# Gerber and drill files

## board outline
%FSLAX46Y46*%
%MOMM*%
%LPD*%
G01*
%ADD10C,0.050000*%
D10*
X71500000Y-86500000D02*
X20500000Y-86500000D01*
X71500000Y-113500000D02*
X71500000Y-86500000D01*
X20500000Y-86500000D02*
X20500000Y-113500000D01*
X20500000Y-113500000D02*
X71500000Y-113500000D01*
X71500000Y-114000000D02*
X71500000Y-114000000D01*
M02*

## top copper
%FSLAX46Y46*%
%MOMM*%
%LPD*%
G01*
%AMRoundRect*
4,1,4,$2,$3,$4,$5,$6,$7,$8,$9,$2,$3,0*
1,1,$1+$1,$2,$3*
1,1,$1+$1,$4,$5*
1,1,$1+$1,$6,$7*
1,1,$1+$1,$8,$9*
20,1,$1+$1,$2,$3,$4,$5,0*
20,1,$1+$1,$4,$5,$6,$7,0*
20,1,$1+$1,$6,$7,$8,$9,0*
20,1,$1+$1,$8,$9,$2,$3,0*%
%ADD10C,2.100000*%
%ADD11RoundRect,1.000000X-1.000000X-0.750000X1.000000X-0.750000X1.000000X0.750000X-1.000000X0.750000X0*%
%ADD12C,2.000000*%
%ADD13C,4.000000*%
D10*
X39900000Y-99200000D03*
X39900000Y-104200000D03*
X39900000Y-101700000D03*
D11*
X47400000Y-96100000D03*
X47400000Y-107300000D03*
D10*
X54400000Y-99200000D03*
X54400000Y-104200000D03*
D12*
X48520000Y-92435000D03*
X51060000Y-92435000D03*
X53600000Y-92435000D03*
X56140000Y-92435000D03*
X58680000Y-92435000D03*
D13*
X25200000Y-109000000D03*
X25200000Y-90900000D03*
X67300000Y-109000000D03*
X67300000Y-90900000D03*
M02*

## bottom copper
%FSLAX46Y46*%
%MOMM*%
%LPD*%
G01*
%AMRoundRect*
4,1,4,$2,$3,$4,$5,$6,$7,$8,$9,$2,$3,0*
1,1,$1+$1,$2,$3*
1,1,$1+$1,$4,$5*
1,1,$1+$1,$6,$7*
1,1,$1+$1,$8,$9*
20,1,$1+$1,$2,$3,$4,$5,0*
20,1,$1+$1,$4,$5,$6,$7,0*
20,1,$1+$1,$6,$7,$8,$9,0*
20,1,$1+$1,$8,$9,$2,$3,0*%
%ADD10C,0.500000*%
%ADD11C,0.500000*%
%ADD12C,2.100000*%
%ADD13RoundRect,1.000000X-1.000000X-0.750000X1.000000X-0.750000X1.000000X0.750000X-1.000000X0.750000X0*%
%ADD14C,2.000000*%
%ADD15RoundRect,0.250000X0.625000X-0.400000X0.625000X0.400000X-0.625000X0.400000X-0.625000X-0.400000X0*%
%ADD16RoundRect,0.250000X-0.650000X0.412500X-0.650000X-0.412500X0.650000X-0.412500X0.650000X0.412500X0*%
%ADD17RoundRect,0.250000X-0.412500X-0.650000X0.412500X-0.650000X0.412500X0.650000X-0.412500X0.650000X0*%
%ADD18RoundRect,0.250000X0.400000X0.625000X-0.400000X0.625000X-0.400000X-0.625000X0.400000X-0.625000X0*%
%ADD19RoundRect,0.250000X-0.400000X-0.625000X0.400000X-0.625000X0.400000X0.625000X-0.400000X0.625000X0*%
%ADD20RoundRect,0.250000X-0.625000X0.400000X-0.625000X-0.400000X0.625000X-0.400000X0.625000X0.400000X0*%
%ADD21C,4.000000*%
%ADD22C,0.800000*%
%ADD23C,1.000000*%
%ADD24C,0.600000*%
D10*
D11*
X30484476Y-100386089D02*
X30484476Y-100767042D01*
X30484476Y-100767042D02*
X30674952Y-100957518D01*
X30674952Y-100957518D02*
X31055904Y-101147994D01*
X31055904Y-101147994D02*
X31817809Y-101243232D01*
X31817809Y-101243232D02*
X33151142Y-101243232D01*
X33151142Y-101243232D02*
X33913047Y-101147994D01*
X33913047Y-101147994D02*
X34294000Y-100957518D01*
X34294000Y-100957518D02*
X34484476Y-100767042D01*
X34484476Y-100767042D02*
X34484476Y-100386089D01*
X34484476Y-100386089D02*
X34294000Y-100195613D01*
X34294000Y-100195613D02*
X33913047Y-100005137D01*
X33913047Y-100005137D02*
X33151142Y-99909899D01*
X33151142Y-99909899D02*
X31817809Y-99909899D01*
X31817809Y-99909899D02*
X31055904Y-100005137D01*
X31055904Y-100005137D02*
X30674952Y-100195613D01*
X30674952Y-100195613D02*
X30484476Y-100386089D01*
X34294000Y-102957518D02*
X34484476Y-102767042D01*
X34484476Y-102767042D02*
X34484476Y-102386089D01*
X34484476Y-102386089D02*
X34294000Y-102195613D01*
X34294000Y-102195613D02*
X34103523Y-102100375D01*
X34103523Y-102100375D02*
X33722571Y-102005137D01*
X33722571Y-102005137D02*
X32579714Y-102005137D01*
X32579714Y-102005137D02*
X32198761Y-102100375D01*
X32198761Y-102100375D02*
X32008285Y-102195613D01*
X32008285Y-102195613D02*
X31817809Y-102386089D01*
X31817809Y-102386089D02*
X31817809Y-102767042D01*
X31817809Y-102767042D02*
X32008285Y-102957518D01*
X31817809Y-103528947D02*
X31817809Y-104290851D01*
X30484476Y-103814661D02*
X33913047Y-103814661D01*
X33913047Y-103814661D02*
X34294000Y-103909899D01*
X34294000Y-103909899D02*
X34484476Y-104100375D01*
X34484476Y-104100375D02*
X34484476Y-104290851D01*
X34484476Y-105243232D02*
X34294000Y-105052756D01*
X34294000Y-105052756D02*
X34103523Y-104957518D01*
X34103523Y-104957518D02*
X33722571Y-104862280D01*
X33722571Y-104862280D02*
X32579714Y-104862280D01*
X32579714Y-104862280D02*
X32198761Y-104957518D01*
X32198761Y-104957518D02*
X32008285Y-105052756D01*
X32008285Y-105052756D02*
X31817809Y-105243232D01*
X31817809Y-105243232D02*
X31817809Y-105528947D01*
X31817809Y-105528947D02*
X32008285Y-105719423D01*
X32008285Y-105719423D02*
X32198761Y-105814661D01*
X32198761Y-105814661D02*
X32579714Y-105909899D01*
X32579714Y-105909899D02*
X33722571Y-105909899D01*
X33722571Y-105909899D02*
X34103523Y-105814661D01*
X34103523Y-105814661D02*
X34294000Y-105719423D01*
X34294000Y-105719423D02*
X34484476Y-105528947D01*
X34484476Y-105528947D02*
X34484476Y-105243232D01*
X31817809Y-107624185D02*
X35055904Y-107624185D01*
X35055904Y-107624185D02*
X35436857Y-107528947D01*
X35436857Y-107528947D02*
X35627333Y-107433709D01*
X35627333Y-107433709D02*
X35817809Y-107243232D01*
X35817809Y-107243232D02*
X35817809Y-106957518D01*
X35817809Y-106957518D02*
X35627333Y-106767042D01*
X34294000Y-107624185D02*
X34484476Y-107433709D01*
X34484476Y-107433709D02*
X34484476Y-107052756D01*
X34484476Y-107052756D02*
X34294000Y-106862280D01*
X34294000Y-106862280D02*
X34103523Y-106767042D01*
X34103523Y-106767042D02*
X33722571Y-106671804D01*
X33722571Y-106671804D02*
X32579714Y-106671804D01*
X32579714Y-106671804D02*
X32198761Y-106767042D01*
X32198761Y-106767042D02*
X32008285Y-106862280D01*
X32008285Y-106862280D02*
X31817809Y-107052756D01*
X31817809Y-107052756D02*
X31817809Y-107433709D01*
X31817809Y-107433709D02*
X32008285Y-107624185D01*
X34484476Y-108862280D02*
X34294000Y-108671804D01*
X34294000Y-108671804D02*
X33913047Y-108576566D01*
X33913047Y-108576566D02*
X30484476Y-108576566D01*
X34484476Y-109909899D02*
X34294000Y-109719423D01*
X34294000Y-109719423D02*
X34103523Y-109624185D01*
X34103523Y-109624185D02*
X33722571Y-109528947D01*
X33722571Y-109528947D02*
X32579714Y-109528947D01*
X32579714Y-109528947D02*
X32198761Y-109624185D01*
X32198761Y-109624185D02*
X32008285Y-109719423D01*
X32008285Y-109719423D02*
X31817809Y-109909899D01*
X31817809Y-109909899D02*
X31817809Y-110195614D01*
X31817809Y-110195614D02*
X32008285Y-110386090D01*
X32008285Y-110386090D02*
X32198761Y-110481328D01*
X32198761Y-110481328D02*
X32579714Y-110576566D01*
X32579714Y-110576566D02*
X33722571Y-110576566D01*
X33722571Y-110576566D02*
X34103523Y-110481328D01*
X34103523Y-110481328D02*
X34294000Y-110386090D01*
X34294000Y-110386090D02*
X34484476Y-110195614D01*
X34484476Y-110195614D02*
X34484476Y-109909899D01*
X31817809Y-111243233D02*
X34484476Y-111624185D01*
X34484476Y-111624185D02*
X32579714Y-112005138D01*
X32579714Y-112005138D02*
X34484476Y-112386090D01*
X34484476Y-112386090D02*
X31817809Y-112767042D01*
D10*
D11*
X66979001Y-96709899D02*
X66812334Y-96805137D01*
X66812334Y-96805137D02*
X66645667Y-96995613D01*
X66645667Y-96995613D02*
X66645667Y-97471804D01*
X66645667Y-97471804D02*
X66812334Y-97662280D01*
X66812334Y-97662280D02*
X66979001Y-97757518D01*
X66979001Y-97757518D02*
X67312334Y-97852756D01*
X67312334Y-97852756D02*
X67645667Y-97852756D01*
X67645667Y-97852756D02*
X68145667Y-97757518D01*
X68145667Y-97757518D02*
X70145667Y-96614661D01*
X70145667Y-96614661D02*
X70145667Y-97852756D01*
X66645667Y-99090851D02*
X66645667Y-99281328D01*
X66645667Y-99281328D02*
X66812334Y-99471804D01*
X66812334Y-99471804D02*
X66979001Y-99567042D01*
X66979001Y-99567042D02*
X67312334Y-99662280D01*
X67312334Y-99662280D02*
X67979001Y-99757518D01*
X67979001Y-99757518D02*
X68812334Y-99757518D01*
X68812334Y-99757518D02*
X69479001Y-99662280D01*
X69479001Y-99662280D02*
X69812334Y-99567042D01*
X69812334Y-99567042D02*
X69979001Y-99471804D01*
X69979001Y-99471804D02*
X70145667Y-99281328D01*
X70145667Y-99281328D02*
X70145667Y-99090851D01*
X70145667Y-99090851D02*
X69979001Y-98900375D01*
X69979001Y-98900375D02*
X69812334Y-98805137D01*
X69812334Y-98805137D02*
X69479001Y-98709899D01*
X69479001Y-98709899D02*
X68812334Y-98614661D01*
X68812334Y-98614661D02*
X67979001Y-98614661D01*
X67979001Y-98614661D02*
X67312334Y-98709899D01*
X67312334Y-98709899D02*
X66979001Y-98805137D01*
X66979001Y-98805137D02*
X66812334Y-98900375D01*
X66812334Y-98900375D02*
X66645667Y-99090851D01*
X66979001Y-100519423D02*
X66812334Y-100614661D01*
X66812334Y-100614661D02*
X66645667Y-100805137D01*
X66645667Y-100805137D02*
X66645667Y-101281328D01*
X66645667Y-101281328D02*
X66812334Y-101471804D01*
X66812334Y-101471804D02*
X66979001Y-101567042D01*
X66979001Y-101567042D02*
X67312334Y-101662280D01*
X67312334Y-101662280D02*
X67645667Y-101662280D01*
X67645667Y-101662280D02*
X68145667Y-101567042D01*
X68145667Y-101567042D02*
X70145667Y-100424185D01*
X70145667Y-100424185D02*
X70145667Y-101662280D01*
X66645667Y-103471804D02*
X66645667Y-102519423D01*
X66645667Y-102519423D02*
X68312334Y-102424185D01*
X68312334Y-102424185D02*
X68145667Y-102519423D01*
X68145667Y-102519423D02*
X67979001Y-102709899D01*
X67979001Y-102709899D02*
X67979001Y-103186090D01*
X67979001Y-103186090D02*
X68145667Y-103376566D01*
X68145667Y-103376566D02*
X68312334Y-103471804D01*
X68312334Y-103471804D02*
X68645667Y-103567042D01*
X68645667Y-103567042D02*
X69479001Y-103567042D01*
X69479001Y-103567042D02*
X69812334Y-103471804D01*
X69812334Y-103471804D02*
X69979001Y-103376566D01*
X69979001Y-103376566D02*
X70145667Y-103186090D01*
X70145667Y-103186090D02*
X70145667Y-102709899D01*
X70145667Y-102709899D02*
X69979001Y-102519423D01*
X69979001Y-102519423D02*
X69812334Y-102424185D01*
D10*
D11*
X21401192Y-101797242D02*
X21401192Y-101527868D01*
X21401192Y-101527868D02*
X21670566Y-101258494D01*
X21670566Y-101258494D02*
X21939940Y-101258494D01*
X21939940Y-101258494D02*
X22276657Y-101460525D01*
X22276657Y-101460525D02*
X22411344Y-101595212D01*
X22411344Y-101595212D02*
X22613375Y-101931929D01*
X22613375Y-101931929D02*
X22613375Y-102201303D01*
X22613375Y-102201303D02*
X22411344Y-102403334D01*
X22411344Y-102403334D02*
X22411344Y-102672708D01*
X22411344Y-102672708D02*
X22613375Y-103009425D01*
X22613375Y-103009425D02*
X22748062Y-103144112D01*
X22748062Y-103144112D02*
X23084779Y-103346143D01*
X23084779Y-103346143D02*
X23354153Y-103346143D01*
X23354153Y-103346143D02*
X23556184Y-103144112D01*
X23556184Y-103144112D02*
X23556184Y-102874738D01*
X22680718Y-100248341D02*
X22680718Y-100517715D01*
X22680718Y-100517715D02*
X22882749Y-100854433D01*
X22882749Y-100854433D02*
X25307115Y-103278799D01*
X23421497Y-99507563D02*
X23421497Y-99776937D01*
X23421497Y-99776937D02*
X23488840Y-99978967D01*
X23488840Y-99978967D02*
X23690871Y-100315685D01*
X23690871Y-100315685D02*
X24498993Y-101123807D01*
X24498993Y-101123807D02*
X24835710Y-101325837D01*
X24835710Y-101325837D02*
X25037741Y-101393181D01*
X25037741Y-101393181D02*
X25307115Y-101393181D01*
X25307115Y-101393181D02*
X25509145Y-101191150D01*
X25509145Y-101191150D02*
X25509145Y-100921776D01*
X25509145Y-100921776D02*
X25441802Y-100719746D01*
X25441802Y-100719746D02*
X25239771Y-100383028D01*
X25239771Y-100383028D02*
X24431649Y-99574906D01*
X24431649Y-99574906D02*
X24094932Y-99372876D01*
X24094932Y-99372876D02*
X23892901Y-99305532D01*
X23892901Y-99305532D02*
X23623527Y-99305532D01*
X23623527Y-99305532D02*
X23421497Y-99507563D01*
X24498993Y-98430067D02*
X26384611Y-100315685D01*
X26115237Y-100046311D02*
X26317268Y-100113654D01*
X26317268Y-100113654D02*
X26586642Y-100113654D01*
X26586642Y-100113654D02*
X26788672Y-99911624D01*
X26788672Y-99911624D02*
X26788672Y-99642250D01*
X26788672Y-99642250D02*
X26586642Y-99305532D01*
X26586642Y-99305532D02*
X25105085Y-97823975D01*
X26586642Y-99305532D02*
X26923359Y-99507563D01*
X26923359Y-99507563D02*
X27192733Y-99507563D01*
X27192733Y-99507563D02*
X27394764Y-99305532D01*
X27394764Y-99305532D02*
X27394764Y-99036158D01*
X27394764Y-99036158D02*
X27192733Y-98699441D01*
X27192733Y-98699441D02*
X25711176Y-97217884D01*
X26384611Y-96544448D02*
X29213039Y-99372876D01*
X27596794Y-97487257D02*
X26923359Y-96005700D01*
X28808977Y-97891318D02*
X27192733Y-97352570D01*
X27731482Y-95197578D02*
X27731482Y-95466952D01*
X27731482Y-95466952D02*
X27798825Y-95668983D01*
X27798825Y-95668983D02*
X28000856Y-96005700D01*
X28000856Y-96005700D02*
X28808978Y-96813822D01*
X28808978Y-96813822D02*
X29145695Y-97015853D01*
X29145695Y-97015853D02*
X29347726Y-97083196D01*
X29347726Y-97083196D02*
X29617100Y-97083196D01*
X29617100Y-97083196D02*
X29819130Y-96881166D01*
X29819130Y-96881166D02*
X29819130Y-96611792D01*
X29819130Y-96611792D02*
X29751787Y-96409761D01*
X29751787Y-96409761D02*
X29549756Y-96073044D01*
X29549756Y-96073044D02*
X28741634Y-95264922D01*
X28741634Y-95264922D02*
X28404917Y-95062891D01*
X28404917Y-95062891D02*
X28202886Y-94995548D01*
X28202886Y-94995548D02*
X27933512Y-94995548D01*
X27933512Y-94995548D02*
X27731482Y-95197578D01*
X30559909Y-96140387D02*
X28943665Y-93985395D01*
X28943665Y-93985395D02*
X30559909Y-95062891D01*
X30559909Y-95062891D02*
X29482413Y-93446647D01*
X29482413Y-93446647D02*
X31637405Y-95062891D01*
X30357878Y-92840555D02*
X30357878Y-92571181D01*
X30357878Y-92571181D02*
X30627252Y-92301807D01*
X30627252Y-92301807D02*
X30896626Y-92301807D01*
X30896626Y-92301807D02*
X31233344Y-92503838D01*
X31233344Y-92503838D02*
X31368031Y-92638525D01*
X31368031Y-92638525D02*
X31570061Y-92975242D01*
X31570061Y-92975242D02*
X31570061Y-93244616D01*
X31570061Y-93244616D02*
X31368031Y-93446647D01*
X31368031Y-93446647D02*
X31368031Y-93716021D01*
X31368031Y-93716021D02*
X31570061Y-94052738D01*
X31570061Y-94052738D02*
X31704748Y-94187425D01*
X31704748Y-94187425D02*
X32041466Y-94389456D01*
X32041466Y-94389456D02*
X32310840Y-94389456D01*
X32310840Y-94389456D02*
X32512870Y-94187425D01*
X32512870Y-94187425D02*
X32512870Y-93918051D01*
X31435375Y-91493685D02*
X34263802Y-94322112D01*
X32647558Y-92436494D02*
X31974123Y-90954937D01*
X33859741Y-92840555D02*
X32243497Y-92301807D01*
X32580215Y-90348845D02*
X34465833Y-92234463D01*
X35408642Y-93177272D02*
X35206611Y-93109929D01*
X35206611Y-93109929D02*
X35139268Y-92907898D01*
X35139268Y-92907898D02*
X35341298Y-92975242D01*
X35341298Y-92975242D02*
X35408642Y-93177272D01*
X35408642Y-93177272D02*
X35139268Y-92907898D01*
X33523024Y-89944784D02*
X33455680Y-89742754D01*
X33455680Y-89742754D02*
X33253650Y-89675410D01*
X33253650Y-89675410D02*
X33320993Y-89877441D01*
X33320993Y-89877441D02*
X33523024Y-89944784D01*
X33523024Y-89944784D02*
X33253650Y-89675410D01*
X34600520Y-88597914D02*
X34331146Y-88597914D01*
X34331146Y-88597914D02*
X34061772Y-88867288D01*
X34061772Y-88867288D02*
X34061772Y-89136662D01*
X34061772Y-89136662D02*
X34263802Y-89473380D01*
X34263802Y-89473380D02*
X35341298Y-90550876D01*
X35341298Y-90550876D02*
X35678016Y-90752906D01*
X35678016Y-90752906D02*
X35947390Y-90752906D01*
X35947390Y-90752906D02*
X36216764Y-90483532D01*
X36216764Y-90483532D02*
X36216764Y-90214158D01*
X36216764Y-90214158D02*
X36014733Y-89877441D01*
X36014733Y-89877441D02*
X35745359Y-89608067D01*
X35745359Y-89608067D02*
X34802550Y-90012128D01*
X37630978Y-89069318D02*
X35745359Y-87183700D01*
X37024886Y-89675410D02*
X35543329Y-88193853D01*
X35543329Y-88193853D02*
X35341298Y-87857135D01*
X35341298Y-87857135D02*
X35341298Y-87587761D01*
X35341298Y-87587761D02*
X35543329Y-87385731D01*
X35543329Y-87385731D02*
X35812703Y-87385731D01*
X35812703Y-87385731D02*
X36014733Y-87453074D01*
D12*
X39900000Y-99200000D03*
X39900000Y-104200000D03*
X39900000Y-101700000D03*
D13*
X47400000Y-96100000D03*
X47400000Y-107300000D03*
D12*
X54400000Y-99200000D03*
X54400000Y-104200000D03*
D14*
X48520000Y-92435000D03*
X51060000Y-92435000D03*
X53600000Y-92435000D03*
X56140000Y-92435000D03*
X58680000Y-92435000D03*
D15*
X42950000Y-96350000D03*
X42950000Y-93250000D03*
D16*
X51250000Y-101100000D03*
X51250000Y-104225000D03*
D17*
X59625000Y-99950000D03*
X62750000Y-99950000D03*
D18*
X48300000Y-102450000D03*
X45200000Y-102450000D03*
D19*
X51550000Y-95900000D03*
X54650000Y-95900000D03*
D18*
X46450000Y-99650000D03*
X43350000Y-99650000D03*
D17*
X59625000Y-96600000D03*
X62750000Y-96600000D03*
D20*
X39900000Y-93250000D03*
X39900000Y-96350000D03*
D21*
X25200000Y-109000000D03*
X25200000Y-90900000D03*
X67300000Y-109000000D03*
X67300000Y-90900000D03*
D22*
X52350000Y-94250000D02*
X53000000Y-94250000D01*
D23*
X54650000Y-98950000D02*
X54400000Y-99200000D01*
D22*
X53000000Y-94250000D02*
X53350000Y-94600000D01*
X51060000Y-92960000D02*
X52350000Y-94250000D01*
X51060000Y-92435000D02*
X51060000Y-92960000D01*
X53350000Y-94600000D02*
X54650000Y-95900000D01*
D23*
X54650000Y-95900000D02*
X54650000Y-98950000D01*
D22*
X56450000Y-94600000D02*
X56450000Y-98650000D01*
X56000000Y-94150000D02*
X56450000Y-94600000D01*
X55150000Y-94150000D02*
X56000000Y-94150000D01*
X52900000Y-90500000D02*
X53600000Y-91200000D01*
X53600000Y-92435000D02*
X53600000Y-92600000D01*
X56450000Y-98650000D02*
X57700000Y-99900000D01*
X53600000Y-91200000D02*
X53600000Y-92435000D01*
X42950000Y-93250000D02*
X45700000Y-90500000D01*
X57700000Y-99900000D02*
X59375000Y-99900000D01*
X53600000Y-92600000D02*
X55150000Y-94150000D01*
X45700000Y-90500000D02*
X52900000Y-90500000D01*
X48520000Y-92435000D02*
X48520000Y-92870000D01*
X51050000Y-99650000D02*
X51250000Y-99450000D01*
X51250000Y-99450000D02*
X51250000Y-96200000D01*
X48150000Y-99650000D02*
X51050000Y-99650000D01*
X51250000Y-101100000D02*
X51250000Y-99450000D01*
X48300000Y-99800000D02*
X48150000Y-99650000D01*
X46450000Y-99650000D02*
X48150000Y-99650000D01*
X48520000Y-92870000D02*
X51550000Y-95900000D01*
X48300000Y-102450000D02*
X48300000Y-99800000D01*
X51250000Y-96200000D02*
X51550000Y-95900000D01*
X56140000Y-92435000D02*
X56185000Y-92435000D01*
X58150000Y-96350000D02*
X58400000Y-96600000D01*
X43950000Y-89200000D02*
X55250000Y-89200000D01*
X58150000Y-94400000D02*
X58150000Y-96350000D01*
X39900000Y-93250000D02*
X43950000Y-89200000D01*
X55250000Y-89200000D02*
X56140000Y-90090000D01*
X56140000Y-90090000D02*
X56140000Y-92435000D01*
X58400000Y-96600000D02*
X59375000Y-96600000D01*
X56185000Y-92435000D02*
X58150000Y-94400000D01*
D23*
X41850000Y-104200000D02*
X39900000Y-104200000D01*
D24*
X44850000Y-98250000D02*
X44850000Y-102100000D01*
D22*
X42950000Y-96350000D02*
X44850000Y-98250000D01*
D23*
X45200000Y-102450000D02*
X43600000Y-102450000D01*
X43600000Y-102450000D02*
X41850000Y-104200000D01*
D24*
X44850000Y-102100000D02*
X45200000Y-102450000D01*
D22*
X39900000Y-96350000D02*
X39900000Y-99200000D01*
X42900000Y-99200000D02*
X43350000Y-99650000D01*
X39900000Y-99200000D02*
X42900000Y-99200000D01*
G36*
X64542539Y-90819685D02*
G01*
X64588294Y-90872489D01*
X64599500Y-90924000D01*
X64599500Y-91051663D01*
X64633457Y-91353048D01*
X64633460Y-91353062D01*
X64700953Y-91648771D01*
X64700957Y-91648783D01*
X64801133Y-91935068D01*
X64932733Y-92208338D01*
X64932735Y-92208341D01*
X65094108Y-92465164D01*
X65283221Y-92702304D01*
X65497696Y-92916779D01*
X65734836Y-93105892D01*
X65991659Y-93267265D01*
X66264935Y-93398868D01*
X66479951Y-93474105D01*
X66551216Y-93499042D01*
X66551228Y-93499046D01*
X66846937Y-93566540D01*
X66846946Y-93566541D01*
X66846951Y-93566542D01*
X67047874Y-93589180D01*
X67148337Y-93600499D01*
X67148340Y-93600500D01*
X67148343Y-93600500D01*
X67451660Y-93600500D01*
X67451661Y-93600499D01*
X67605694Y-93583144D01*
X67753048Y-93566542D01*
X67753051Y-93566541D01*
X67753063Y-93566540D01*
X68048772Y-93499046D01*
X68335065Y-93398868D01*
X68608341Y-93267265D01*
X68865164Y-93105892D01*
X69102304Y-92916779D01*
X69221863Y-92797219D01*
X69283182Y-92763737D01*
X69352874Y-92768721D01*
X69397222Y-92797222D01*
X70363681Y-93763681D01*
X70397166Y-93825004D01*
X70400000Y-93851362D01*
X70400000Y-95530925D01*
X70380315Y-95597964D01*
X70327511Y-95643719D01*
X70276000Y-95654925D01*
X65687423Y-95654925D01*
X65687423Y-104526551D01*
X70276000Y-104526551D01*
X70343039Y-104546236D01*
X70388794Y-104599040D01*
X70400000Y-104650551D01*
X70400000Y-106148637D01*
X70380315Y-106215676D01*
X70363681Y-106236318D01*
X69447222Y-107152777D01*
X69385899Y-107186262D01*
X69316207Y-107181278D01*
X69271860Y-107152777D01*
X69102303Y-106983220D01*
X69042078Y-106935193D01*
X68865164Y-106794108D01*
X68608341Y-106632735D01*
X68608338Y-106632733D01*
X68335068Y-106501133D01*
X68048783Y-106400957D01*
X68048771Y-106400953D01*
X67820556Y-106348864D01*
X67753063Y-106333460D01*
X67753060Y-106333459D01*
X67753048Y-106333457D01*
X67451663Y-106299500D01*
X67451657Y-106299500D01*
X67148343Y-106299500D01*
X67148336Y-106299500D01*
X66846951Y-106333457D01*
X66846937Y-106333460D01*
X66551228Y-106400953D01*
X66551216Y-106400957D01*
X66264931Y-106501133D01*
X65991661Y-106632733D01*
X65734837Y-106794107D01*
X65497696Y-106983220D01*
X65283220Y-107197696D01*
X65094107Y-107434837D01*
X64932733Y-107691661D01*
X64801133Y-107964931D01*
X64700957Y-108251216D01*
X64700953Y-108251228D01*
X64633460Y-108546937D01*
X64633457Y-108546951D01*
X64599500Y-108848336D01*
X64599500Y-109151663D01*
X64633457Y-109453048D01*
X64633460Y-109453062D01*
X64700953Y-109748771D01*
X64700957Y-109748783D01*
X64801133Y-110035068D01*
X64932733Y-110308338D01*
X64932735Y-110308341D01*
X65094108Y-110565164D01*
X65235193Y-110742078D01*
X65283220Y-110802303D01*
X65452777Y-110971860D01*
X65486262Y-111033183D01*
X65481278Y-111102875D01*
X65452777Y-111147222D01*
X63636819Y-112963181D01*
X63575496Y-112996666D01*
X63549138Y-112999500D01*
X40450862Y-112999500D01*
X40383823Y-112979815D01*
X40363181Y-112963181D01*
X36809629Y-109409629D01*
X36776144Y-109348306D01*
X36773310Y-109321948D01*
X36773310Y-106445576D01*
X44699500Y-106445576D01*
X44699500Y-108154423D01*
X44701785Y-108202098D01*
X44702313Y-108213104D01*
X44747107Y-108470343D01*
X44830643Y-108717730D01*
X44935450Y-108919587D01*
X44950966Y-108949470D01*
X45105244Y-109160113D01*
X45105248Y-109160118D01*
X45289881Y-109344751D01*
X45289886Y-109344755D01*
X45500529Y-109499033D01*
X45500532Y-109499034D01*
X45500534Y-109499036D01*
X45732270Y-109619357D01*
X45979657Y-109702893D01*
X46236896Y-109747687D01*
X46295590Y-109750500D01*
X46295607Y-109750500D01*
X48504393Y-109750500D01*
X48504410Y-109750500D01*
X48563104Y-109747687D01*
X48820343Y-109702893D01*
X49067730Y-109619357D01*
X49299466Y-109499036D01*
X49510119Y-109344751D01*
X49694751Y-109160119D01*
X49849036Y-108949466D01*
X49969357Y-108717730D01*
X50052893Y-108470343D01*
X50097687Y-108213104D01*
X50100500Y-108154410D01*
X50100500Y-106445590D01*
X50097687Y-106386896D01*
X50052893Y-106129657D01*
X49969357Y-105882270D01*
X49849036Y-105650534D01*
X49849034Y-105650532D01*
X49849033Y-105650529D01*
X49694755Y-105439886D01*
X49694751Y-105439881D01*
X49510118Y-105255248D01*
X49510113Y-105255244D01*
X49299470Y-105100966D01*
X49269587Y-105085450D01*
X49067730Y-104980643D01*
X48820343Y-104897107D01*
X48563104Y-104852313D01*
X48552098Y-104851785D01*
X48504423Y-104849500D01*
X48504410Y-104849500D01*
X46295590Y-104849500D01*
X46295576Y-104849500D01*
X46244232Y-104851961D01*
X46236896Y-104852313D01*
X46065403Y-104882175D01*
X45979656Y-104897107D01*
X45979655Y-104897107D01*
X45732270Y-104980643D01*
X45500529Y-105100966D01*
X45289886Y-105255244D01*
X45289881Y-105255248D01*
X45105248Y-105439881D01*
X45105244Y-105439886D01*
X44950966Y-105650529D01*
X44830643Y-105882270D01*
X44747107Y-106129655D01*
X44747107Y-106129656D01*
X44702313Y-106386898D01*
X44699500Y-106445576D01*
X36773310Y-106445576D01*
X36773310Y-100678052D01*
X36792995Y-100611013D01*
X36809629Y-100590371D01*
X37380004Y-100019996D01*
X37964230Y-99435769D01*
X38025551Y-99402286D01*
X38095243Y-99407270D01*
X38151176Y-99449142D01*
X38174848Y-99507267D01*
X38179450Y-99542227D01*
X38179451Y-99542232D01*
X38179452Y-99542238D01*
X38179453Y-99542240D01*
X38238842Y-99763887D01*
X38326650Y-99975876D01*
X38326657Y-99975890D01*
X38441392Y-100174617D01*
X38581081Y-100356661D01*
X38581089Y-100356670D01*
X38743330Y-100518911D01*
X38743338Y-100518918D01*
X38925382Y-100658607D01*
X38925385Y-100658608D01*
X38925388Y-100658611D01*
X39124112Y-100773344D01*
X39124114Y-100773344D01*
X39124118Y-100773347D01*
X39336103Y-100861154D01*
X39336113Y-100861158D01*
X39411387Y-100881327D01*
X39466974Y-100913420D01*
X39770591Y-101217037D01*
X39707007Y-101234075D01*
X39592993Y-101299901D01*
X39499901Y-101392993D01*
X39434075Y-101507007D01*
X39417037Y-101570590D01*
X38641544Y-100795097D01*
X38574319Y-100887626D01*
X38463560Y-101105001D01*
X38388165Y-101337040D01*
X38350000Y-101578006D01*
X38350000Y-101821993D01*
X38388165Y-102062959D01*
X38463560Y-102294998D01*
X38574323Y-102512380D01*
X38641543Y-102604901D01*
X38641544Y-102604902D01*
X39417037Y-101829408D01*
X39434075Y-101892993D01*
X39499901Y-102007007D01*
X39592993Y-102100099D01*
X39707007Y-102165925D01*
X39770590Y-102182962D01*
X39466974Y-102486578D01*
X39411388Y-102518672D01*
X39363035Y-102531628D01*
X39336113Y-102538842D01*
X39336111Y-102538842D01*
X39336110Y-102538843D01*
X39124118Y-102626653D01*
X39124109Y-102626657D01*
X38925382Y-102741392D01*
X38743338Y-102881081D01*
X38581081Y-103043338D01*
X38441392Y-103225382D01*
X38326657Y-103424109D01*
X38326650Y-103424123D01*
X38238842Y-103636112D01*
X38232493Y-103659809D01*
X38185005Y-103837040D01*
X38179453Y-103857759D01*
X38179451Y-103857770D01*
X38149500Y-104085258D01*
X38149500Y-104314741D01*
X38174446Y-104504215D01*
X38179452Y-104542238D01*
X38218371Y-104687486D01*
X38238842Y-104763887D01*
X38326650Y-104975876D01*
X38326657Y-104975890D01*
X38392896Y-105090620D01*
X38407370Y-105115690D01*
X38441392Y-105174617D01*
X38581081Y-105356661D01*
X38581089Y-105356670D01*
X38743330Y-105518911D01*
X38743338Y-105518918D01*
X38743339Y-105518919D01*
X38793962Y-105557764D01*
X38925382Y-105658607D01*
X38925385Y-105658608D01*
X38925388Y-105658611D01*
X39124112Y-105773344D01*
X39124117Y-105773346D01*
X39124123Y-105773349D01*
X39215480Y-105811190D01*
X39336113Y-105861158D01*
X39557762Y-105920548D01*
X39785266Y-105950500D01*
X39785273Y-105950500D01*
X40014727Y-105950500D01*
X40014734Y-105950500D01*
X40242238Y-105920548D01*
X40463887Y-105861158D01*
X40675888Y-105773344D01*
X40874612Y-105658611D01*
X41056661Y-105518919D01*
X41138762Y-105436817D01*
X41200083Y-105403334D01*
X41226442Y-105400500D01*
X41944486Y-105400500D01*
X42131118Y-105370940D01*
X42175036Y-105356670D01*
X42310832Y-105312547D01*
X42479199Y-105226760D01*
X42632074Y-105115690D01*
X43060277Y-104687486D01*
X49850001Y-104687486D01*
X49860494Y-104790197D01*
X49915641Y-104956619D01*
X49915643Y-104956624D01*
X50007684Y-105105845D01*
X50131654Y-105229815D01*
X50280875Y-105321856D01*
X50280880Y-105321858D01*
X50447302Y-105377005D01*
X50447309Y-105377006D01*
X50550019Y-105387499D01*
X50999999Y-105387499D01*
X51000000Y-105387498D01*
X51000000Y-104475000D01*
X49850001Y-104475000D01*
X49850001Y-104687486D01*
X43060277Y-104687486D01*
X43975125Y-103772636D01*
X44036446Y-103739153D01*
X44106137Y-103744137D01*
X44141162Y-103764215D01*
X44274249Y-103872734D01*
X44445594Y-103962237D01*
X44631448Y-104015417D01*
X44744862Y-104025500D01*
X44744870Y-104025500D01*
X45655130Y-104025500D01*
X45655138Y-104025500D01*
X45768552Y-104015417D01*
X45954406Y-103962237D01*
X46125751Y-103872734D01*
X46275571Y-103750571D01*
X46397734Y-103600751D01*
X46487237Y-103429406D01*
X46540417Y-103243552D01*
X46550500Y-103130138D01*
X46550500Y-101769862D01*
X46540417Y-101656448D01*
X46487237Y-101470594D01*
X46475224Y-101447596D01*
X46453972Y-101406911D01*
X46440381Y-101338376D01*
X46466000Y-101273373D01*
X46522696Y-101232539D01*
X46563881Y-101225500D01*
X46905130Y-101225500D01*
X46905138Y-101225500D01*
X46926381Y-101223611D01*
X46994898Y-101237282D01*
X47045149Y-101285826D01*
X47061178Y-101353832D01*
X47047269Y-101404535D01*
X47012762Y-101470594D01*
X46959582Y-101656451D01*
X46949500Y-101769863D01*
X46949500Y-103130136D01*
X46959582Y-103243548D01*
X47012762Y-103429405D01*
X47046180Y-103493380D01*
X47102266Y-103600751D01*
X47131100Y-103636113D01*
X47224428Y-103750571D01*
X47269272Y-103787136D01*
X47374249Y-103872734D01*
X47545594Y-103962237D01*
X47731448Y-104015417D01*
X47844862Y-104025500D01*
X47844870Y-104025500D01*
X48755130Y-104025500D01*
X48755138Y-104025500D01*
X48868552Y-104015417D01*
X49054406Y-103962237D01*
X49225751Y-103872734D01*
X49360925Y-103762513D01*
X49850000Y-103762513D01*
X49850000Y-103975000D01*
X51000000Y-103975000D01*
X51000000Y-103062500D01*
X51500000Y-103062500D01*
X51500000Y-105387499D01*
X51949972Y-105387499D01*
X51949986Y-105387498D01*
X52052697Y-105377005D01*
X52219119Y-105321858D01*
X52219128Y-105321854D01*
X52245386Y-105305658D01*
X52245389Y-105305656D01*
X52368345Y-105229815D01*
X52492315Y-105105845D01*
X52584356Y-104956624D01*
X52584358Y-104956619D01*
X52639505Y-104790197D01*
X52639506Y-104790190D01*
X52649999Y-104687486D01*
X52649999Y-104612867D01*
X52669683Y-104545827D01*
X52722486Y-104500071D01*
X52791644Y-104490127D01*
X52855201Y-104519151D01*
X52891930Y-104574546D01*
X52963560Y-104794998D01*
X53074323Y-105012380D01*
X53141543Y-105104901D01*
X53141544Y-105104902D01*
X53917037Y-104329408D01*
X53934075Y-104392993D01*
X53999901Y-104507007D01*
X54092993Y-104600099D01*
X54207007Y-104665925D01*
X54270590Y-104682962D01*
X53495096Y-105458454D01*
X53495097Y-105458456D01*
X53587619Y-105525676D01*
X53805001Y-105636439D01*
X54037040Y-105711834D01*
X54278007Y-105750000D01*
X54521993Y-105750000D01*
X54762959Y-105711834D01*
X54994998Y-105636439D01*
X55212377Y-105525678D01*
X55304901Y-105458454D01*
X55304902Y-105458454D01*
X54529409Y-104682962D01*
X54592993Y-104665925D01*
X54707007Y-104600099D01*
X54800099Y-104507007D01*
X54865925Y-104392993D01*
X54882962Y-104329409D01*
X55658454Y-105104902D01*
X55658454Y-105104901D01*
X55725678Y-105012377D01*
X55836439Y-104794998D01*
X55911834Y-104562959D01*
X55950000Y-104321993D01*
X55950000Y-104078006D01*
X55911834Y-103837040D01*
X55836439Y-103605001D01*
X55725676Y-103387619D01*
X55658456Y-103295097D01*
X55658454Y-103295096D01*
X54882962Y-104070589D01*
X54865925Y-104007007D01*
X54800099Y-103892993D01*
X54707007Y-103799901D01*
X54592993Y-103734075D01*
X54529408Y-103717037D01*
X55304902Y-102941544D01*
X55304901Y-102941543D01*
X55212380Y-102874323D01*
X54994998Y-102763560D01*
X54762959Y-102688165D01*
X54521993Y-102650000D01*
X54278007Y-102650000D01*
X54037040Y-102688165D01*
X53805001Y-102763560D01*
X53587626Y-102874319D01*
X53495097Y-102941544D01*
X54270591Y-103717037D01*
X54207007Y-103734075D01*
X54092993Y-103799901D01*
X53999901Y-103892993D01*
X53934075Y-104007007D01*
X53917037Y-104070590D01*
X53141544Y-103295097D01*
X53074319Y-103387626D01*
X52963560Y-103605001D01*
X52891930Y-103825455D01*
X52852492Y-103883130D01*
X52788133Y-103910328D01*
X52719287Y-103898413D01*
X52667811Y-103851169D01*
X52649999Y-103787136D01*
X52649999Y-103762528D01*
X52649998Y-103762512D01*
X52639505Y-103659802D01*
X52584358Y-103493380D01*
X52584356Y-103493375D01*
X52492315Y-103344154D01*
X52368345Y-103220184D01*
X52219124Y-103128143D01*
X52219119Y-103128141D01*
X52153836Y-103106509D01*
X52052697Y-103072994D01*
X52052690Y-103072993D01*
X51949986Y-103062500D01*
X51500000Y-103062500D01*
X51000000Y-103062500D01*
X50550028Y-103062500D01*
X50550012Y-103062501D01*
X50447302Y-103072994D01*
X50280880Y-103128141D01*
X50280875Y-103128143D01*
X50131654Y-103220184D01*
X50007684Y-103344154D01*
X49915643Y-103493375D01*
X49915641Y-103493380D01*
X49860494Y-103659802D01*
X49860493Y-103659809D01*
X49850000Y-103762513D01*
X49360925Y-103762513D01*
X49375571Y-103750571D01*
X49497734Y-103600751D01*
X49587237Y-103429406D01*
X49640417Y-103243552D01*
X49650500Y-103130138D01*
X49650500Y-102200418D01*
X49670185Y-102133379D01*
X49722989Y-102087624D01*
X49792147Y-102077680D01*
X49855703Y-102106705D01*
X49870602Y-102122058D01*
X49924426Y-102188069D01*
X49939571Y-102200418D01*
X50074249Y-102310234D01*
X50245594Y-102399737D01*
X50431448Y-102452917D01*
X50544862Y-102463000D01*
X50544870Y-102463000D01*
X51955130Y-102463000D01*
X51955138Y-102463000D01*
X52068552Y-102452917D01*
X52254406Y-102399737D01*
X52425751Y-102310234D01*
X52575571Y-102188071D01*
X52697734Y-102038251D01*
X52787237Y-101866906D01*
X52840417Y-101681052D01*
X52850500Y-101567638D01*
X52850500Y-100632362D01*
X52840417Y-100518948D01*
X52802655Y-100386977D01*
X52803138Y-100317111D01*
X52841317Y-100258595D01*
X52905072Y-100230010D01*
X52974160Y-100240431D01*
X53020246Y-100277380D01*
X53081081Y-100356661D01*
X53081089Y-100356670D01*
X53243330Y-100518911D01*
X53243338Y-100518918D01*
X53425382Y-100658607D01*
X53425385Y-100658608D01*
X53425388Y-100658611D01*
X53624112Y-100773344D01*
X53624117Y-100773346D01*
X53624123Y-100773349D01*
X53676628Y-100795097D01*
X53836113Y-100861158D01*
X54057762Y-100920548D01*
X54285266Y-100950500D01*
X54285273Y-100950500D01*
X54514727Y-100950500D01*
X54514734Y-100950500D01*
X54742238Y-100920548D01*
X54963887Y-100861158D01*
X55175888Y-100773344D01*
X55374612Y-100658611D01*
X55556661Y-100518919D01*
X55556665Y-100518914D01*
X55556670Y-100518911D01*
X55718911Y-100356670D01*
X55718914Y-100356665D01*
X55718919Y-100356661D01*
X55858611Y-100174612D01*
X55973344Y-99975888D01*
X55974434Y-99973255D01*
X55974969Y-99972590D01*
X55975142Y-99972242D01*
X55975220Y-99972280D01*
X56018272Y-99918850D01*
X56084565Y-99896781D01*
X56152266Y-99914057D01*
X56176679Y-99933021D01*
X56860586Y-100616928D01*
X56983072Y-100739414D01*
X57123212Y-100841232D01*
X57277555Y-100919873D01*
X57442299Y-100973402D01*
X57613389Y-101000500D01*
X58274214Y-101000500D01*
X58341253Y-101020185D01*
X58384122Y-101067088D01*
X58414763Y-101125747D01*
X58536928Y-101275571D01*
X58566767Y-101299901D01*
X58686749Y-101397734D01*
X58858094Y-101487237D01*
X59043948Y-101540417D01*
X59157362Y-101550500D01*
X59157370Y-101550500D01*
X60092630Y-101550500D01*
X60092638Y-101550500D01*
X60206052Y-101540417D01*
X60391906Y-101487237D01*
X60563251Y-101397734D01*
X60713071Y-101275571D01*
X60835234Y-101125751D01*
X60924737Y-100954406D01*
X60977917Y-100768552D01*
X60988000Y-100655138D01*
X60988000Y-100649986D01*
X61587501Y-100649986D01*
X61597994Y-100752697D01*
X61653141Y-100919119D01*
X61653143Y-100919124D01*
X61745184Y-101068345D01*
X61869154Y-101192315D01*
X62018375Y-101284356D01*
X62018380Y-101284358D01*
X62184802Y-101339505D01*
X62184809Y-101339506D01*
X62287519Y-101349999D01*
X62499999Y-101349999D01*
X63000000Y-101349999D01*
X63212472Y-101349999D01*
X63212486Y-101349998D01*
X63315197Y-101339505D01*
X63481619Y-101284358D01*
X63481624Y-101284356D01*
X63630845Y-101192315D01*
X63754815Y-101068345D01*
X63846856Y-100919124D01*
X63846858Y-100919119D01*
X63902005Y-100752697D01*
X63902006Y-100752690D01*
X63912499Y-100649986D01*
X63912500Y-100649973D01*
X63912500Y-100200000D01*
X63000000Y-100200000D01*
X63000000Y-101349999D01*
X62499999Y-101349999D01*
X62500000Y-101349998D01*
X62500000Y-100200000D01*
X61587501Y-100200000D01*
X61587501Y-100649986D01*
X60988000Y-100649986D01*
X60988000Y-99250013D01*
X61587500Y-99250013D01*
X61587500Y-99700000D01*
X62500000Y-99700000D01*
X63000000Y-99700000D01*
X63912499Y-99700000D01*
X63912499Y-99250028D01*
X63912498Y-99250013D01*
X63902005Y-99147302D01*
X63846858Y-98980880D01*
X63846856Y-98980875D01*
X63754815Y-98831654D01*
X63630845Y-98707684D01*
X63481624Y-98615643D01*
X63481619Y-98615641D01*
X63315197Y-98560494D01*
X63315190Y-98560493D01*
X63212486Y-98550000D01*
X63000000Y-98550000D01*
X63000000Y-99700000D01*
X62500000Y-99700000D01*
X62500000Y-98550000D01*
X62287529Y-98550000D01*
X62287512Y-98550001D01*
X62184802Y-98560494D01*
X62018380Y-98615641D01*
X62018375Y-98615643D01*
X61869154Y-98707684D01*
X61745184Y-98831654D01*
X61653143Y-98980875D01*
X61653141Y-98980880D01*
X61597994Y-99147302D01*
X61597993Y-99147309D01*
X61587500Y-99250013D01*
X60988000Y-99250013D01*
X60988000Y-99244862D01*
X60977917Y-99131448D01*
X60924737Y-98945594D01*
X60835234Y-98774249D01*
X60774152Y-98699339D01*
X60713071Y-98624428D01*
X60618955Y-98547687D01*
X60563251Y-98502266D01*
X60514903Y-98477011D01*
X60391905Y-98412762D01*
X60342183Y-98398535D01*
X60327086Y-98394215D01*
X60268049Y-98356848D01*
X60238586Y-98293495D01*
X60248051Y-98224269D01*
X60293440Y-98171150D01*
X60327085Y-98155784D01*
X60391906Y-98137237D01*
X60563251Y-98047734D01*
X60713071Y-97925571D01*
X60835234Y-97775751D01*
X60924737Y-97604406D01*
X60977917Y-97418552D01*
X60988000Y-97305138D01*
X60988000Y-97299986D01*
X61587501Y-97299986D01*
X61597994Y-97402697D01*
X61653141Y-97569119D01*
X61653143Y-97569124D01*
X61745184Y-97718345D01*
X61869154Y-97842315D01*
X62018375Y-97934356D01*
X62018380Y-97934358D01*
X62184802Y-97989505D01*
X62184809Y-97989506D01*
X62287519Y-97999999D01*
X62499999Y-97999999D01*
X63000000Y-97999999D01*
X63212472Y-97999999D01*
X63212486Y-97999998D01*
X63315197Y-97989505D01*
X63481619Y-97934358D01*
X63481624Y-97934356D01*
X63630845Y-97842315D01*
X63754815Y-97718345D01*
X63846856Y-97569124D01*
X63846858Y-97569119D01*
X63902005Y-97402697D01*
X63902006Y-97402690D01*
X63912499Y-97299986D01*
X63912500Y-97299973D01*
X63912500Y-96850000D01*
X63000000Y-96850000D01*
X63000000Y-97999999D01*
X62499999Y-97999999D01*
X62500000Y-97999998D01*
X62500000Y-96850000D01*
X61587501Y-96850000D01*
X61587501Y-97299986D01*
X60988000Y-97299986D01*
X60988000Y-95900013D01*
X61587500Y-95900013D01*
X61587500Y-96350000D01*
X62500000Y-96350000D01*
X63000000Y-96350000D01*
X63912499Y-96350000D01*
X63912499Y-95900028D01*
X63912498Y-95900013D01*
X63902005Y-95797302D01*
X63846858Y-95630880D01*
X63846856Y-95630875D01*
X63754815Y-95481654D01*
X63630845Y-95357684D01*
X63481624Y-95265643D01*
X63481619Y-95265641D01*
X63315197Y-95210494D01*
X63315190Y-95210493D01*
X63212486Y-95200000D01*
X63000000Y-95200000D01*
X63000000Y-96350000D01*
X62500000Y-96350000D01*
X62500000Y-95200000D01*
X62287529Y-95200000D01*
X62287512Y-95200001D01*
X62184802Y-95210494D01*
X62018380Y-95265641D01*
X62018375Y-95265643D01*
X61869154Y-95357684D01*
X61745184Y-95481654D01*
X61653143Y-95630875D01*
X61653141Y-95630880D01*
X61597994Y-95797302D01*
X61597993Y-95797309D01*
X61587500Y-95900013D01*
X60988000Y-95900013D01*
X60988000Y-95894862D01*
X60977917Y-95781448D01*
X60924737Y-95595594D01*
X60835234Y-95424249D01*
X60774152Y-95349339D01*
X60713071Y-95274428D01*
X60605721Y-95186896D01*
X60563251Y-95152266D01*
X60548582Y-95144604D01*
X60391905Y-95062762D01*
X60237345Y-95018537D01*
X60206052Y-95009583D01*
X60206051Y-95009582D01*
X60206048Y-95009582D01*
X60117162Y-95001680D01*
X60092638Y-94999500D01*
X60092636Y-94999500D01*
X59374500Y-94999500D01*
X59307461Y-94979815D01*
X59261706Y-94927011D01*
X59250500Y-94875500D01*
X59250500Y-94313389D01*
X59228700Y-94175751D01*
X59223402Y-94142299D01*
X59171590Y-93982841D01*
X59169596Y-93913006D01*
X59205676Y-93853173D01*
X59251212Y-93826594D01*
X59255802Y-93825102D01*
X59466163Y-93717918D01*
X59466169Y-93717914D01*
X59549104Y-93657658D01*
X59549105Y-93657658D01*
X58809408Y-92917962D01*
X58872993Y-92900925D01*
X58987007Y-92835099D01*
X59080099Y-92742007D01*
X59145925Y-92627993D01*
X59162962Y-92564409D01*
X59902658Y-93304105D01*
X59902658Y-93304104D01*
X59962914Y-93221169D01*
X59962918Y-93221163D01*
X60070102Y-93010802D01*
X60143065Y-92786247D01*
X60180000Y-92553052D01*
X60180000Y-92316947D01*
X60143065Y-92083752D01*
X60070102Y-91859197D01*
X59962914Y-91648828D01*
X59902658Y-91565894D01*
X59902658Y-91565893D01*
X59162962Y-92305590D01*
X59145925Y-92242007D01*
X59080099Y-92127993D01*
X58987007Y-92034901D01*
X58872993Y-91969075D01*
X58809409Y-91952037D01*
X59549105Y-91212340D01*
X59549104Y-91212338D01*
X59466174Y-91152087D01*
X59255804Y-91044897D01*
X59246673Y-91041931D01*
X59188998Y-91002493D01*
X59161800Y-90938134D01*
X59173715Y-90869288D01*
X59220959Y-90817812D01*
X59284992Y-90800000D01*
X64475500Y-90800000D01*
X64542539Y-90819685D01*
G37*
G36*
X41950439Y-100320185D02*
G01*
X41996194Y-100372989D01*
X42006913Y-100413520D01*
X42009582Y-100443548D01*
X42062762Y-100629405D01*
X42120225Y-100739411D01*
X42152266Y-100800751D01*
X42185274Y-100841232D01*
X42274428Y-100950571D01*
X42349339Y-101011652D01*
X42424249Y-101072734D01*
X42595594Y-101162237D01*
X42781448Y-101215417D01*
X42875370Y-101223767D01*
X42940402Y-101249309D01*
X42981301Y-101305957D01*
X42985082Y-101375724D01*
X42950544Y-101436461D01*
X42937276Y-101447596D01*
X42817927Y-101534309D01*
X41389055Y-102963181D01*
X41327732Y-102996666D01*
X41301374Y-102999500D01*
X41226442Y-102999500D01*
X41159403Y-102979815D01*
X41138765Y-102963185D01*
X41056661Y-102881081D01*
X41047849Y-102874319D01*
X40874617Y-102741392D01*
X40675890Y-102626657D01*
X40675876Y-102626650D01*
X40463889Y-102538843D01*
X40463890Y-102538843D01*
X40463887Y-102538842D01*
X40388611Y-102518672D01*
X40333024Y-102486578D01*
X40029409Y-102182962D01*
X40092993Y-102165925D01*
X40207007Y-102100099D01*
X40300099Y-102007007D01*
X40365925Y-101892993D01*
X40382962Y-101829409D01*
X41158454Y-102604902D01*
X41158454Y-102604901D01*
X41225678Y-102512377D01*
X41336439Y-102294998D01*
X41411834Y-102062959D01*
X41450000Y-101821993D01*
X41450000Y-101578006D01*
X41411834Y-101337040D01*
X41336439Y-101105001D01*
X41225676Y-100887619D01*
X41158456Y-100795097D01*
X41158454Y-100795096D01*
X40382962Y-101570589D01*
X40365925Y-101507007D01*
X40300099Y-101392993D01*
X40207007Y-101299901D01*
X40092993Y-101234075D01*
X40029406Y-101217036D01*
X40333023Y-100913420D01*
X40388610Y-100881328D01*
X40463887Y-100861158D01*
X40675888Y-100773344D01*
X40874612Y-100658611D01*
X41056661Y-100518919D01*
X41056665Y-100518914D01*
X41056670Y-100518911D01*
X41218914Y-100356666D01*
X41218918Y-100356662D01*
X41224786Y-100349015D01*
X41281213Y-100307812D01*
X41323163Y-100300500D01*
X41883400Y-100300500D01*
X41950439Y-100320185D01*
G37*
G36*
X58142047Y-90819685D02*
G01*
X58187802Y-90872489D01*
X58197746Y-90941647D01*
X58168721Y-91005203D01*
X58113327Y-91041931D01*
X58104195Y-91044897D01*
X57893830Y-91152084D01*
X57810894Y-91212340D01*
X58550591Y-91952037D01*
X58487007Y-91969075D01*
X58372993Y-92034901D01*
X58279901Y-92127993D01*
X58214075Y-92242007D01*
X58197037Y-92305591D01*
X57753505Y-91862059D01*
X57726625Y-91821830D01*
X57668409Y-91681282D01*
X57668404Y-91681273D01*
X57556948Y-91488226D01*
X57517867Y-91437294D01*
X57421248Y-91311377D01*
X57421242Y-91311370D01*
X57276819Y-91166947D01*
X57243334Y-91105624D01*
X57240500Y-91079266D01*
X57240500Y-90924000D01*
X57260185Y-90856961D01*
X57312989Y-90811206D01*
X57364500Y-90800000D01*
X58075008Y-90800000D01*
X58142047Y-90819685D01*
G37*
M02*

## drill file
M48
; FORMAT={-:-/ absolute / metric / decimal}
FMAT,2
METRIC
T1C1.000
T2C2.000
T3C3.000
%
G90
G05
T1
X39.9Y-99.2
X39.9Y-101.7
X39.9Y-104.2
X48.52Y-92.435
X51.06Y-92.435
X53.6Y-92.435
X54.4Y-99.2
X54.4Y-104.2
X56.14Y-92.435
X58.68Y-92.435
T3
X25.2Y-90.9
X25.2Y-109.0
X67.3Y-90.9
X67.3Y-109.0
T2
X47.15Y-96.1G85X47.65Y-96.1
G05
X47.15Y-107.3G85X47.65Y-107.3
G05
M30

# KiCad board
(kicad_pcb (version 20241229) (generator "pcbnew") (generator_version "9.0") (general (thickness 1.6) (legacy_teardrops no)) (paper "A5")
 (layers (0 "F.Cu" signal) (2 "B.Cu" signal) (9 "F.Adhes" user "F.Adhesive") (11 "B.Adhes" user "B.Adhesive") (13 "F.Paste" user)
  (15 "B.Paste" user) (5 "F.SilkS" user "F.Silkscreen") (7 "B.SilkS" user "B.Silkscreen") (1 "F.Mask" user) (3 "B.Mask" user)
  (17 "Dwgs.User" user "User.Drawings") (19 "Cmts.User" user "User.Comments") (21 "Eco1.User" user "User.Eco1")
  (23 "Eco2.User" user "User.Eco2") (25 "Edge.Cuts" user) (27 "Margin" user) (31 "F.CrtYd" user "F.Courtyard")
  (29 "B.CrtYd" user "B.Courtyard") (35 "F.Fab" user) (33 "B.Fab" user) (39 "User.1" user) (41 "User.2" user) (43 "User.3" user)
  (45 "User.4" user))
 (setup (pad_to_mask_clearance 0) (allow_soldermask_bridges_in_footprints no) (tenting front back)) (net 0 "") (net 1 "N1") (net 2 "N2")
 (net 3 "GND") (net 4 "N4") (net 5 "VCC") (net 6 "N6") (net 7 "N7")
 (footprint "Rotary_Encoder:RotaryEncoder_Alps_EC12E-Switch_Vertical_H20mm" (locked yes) (layer "F.Cu") (at 39.9 99.2)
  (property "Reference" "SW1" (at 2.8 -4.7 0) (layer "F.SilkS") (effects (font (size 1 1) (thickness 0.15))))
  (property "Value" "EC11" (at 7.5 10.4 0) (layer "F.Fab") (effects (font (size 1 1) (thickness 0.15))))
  (pad "A" thru_hole circle (at 0 0) (size 2.1 2.1) (drill 1) (layers "*.Cu" "*.Mask") (remove_unused_layers no) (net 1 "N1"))
  (pad "B" thru_hole circle (at 0 5) (size 2.1 2.1) (drill 1) (layers "*.Cu" "*.Mask") (remove_unused_layers no) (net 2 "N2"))
  (pad "C" thru_hole circle (at 0 2.5) (size 2.1 2.1) (drill 1) (layers "*.Cu" "*.Mask") (remove_unused_layers no) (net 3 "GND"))
  (pad "MP" thru_hole roundrect (at 7.5 -3.1) (size 4 3.5) (drill oval 2.5 2) (layers "*.Cu" "*.Mask") (remove_unused_layers no)
   (roundrect_rratio 0.2857142857))
  (pad "MP" thru_hole roundrect (at 7.5 8.1) (size 4 3.5) (drill oval 2.5 2) (layers "*.Cu" "*.Mask") (remove_unused_layers no)
   (roundrect_rratio 0.2857142857))
  (pad "S1" thru_hole circle (at 14.5 0) (size 2.1 2.1) (drill 1) (layers "*.Cu" "*.Mask") (remove_unused_layers no) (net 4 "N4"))
  (pad "S2" thru_hole circle (at 14.5 5) (size 2.1 2.1) (drill 1) (layers "*.Cu" "*.Mask") (remove_unused_layers no) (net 3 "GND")))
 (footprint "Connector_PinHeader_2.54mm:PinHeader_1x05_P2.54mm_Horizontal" (layer "F.Cu") (at 48.52 92.435 90)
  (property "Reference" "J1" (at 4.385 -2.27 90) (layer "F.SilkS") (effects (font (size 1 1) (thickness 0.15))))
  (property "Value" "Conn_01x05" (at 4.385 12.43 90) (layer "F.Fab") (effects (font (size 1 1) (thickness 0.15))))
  (pad "1" thru_hole circle (at 0 0 90) (size 2 2) (drill 1) (layers "*.Cu" "*.Mask") (remove_unused_layers no) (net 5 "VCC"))
  (pad "2" thru_hole circle (at 0 2.54 90) (size 2 2) (drill 1) (layers "*.Cu" "*.Mask") (remove_unused_layers no) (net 4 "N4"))
  (pad "3" thru_hole circle (at 0 5.08 90) (size 2 2) (drill 1) (layers "*.Cu" "*.Mask") (remove_unused_layers no) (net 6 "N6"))
  (pad "4" thru_hole circle (at 0 7.62 90) (size 2 2) (drill 1) (layers "*.Cu" "*.Mask") (remove_unused_layers no) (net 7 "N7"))
  (pad "5" thru_hole circle (at 0 10.16 90) (size 2 2) (drill 1) (layers "*.Cu" "*.Mask") (remove_unused_layers no) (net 3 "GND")))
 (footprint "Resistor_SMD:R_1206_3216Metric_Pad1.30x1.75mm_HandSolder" (layer "B.Cu") (at 42.95 94.8 90)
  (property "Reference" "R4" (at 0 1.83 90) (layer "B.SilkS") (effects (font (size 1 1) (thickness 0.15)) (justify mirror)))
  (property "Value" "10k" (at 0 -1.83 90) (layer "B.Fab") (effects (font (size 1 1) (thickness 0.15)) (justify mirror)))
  (pad "1" smd roundrect (at -1.55 0 90) (size 1.3 1.75) (layers "B.Cu" "B.Mask" "B.Paste") (roundrect_rratio 0.192308) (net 2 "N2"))
  (pad "2" smd roundrect (at 1.55 0 90) (size 1.3 1.75) (layers "B.Cu" "B.Mask" "B.Paste") (roundrect_rratio 0.192308) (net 6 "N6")))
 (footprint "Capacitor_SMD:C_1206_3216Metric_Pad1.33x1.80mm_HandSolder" (layer "B.Cu") (at 51.25 102.6625 -90)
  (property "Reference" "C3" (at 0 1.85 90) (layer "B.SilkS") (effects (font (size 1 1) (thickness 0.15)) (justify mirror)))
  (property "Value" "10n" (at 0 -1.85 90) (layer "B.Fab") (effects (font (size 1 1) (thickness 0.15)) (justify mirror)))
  (pad "1" smd roundrect (at -1.5625 0 270) (size 1.325 1.8) (layers "B.Cu" "B.Mask" "B.Paste") (roundrect_rratio 0.188679) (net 5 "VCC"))
  (pad "2" smd roundrect (at 1.5625 0 270) (size 1.325 1.8) (layers "B.Cu" "B.Mask" "B.Paste") (roundrect_rratio 0.188679) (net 3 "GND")))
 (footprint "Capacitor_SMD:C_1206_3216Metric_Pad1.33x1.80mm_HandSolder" (layer "B.Cu") (at 61.1875 99.95)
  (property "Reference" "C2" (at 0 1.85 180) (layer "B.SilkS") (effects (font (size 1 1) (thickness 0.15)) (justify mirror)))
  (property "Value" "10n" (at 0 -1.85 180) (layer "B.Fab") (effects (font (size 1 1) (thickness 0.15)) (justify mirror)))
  (pad "1" smd roundrect (at -1.5625 0) (size 1.325 1.8) (layers "B.Cu" "B.Mask" "B.Paste") (roundrect_rratio 0.188679) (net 6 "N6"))
  (pad "2" smd roundrect (at 1.5625 0) (size 1.325 1.8) (layers "B.Cu" "B.Mask" "B.Paste") (roundrect_rratio 0.188679) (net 3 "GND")))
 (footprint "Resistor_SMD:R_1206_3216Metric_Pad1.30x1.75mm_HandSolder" (layer "B.Cu") (at 46.75 102.45 180)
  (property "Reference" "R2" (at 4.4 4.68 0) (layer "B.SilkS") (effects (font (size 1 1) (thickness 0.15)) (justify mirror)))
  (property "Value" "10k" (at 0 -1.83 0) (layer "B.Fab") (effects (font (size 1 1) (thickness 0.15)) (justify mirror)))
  (pad "1" smd roundrect (at -1.55 0 180) (size 1.3 1.75) (layers "B.Cu" "B.Mask" "B.Paste") (roundrect_rratio 0.192308) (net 5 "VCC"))
  (pad "2" smd roundrect (at 1.55 0 180) (size 1.3 1.75) (layers "B.Cu" "B.Mask" "B.Paste") (roundrect_rratio 0.192308) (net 2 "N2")))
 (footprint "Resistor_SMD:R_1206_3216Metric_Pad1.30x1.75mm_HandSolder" (layer "B.Cu") (at 53.1 95.9)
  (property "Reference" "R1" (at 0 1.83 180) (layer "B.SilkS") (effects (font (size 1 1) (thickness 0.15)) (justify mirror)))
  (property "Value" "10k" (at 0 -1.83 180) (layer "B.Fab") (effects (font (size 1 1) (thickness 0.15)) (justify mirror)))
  (pad "1" smd roundrect (at -1.55 0) (size 1.3 1.75) (layers "B.Cu" "B.Mask" "B.Paste") (roundrect_rratio 0.192308) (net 5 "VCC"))
  (pad "2" smd roundrect (at 1.55 0) (size 1.3 1.75) (layers "B.Cu" "B.Mask" "B.Paste") (roundrect_rratio 0.192308) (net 4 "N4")))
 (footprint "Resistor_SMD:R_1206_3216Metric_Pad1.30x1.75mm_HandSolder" (layer "B.Cu") (at 44.9 99.65 180)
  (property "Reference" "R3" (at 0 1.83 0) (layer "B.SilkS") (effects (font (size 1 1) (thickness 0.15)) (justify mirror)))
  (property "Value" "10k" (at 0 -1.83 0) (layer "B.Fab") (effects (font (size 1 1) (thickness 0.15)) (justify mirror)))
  (pad "1" smd roundrect (at -1.55 0 180) (size 1.3 1.75) (layers "B.Cu" "B.Mask" "B.Paste") (roundrect_rratio 0.192308) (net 5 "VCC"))
  (pad "2" smd roundrect (at 1.55 0 180) (size 1.3 1.75) (layers "B.Cu" "B.Mask" "B.Paste") (roundrect_rratio 0.192308) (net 1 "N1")))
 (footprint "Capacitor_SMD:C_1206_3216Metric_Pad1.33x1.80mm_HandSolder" (layer "B.Cu") (at 61.1875 96.6)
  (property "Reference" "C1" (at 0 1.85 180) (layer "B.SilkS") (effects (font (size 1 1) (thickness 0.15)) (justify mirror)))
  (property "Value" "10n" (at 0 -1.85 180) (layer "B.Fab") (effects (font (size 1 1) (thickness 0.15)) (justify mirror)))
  (pad "1" smd roundrect (at -1.5625 0) (size 1.325 1.8) (layers "B.Cu" "B.Mask" "B.Paste") (roundrect_rratio 0.188679) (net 7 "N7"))
  (pad "2" smd roundrect (at 1.5625 0) (size 1.325 1.8) (layers "B.Cu" "B.Mask" "B.Paste") (roundrect_rratio 0.188679) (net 3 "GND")))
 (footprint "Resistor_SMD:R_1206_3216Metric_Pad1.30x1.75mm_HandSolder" (layer "B.Cu") (at 39.9 94.8 -90)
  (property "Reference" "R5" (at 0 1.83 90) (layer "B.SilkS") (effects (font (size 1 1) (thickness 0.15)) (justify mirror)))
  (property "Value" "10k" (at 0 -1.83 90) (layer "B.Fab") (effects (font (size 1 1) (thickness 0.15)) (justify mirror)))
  (pad "1" smd roundrect (at -1.55 0 270) (size 1.3 1.75) (layers "B.Cu" "B.Mask" "B.Paste") (roundrect_rratio 0.192308) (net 7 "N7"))
  (pad "2" smd roundrect (at 1.55 0 270) (size 1.3 1.75) (layers "B.Cu" "B.Mask" "B.Paste") (roundrect_rratio 0.192308) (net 1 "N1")))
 (gr_line (start 71.5 86.5) (end 20.5 86.5) (stroke (width 0.05) (type default)) (layer "Edge.Cuts"))
 (gr_line (start 71.5 113.5) (end 71.5 86.5) (stroke (width 0.05) (type default)) (layer "Edge.Cuts"))
 (gr_line (start 20.5 86.5) (end 20.5 113.5) (stroke (width 0.05) (type default)) (layer "Edge.Cuts"))
 (gr_line (start 20.5 113.5) (end 71.5 113.5) (stroke (width 0.05) (type default)) (layer "Edge.Cuts"))
 (gr_line (start 71.5 114) (end 71.5 114) (stroke (width 0.05) (type default)) (layer "Edge.Cuts"))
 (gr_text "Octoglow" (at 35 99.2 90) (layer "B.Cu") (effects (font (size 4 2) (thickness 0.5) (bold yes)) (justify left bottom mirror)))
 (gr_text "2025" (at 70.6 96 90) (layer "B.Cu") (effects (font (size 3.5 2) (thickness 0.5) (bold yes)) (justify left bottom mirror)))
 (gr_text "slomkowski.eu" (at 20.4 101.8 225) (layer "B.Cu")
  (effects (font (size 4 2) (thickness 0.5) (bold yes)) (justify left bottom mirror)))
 (via (at 25.2 109) (size 4) (drill 3) (layers "F.Cu" "B.Cu") (locked yes) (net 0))
 (via (at 25.2 90.9) (size 4) (drill 3) (layers "F.Cu" "B.Cu") (locked yes) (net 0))
 (via (at 67.3 109) (size 4) (drill 3) (layers "F.Cu" "B.Cu") (locked yes) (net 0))
 (via (at 67.3 90.9) (size 4) (drill 3) (layers "F.Cu" "B.Cu") (locked yes) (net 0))
 (segment (start 52.35 94.25) (end 53 94.25) (width 0.8) (layer "B.Cu") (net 4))
 (segment (start 54.65 98.95) (end 54.4 99.2) (width 1) (layer "B.Cu") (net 4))
 (segment (start 53 94.25) (end 53.35 94.6) (width 0.8) (layer "B.Cu") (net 4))
 (segment (start 51.06 92.96) (end 52.35 94.25) (width 0.8) (layer "B.Cu") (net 4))
 (segment (start 51.06 92.435) (end 51.06 92.96) (width 0.8) (layer "B.Cu") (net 4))
 (segment (start 53.35 94.6) (end 54.65 95.9) (width 0.8) (layer "B.Cu") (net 4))
 (segment (start 54.65 95.9) (end 54.65 98.95) (width 1) (layer "B.Cu") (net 4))
 (segment (start 56.45 94.6) (end 56.45 98.65) (width 0.8) (layer "B.Cu") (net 6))
 (segment (start 56 94.15) (end 56.45 94.6) (width 0.8) (layer "B.Cu") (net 6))
 (segment (start 55.15 94.15) (end 56 94.15) (width 0.8) (layer "B.Cu") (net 6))
 (segment (start 52.9 90.5) (end 53.6 91.2) (width 0.8) (layer "B.Cu") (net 6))
 (segment (start 53.6 92.435) (end 53.6 92.6) (width 0.8) (layer "B.Cu") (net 6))
 (segment (start 56.45 98.65) (end 57.7 99.9) (width 0.8) (layer "B.Cu") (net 6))
 (segment (start 53.6 91.2) (end 53.6 92.435) (width 0.8) (layer "B.Cu") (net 6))
 (segment (start 42.95 93.25) (end 45.7 90.5) (width 0.8) (layer "B.Cu") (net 6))
 (segment (start 57.7 99.9) (end 59.375 99.9) (width 0.8) (layer "B.Cu") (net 6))
 (segment (start 53.6 92.6) (end 55.15 94.15) (width 0.8) (layer "B.Cu") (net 6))
 (segment (start 45.7 90.5) (end 52.9 90.5) (width 0.8) (layer "B.Cu") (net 6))
 (segment (start 48.52 92.435) (end 48.52 92.87) (width 0.8) (layer "B.Cu") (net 5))
 (segment (start 51.05 99.65) (end 51.25 99.45) (width 0.8) (layer "B.Cu") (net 5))
 (segment (start 51.25 99.45) (end 51.25 96.2) (width 0.8) (layer "B.Cu") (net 5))
 (segment (start 48.15 99.65) (end 51.05 99.65) (width 0.8) (layer "B.Cu") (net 5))
 (segment (start 51.25 101.1) (end 51.25 99.45) (width 0.8) (layer "B.Cu") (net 5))
 (segment (start 48.3 99.8) (end 48.15 99.65) (width 0.8) (layer "B.Cu") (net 5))
 (segment (start 46.45 99.65) (end 48.15 99.65) (width 0.8) (layer "B.Cu") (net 5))
 (segment (start 48.52 92.87) (end 51.55 95.9) (width 0.8) (layer "B.Cu") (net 5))
 (segment (start 48.3 102.45) (end 48.3 99.8) (width 0.8) (layer "B.Cu") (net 5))
 (segment (start 51.25 96.2) (end 51.55 95.9) (width 0.8) (layer "B.Cu") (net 5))
 (segment (start 56.14 92.435) (end 56.185 92.435) (width 0.8) (layer "B.Cu") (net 7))
 (segment (start 58.15 96.35) (end 58.4 96.6) (width 0.8) (layer "B.Cu") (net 7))
 (segment (start 43.95 89.2) (end 55.25 89.2) (width 0.8) (layer "B.Cu") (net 7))
 (segment (start 58.15 94.4) (end 58.15 96.35) (width 0.8) (layer "B.Cu") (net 7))
 (segment (start 39.9 93.25) (end 43.95 89.2) (width 0.8) (layer "B.Cu") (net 7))
 (segment (start 55.25 89.2) (end 56.14 90.09) (width 0.8) (layer "B.Cu") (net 7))
 (segment (start 56.14 90.09) (end 56.14 92.435) (width 0.8) (layer "B.Cu") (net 7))
 (segment (start 58.4 96.6) (end 59.375 96.6) (width 0.8) (layer "B.Cu") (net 7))
 (segment (start 56.185 92.435) (end 58.15 94.4) (width 0.8) (layer "B.Cu") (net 7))
 (segment (start 41.85 104.2) (end 39.9 104.2) (width 1) (layer "B.Cu") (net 2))
 (segment (start 44.85 98.25) (end 44.85 102.1) (width 0.6) (layer "B.Cu") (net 2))
 (segment (start 42.95 96.35) (end 44.85 98.25) (width 0.8) (layer "B.Cu") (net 2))
 (segment (start 45.2 102.45) (end 43.6 102.45) (width 1) (layer "B.Cu") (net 2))
 (segment (start 43.6 102.45) (end 41.85 104.2) (width 1) (layer "B.Cu") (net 2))
 (segment (start 44.85 102.1) (end 45.2 102.45) (width 0.6) (layer "B.Cu") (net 2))
 (segment (start 39.9 96.35) (end 39.9 99.2) (width 0.8) (layer "B.Cu") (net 1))
 (segment (start 42.9 99.2) (end 43.35 99.65) (width 0.8) (layer "B.Cu") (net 1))
 (segment (start 39.9 99.2) (end 42.9 99.2) (width 0.8) (layer "B.Cu") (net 1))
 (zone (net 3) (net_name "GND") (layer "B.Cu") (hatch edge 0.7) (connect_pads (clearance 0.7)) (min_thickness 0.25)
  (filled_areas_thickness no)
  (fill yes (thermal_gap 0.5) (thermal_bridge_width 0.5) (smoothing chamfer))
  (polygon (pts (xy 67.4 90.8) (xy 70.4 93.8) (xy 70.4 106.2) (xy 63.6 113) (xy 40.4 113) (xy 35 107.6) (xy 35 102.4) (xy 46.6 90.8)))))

